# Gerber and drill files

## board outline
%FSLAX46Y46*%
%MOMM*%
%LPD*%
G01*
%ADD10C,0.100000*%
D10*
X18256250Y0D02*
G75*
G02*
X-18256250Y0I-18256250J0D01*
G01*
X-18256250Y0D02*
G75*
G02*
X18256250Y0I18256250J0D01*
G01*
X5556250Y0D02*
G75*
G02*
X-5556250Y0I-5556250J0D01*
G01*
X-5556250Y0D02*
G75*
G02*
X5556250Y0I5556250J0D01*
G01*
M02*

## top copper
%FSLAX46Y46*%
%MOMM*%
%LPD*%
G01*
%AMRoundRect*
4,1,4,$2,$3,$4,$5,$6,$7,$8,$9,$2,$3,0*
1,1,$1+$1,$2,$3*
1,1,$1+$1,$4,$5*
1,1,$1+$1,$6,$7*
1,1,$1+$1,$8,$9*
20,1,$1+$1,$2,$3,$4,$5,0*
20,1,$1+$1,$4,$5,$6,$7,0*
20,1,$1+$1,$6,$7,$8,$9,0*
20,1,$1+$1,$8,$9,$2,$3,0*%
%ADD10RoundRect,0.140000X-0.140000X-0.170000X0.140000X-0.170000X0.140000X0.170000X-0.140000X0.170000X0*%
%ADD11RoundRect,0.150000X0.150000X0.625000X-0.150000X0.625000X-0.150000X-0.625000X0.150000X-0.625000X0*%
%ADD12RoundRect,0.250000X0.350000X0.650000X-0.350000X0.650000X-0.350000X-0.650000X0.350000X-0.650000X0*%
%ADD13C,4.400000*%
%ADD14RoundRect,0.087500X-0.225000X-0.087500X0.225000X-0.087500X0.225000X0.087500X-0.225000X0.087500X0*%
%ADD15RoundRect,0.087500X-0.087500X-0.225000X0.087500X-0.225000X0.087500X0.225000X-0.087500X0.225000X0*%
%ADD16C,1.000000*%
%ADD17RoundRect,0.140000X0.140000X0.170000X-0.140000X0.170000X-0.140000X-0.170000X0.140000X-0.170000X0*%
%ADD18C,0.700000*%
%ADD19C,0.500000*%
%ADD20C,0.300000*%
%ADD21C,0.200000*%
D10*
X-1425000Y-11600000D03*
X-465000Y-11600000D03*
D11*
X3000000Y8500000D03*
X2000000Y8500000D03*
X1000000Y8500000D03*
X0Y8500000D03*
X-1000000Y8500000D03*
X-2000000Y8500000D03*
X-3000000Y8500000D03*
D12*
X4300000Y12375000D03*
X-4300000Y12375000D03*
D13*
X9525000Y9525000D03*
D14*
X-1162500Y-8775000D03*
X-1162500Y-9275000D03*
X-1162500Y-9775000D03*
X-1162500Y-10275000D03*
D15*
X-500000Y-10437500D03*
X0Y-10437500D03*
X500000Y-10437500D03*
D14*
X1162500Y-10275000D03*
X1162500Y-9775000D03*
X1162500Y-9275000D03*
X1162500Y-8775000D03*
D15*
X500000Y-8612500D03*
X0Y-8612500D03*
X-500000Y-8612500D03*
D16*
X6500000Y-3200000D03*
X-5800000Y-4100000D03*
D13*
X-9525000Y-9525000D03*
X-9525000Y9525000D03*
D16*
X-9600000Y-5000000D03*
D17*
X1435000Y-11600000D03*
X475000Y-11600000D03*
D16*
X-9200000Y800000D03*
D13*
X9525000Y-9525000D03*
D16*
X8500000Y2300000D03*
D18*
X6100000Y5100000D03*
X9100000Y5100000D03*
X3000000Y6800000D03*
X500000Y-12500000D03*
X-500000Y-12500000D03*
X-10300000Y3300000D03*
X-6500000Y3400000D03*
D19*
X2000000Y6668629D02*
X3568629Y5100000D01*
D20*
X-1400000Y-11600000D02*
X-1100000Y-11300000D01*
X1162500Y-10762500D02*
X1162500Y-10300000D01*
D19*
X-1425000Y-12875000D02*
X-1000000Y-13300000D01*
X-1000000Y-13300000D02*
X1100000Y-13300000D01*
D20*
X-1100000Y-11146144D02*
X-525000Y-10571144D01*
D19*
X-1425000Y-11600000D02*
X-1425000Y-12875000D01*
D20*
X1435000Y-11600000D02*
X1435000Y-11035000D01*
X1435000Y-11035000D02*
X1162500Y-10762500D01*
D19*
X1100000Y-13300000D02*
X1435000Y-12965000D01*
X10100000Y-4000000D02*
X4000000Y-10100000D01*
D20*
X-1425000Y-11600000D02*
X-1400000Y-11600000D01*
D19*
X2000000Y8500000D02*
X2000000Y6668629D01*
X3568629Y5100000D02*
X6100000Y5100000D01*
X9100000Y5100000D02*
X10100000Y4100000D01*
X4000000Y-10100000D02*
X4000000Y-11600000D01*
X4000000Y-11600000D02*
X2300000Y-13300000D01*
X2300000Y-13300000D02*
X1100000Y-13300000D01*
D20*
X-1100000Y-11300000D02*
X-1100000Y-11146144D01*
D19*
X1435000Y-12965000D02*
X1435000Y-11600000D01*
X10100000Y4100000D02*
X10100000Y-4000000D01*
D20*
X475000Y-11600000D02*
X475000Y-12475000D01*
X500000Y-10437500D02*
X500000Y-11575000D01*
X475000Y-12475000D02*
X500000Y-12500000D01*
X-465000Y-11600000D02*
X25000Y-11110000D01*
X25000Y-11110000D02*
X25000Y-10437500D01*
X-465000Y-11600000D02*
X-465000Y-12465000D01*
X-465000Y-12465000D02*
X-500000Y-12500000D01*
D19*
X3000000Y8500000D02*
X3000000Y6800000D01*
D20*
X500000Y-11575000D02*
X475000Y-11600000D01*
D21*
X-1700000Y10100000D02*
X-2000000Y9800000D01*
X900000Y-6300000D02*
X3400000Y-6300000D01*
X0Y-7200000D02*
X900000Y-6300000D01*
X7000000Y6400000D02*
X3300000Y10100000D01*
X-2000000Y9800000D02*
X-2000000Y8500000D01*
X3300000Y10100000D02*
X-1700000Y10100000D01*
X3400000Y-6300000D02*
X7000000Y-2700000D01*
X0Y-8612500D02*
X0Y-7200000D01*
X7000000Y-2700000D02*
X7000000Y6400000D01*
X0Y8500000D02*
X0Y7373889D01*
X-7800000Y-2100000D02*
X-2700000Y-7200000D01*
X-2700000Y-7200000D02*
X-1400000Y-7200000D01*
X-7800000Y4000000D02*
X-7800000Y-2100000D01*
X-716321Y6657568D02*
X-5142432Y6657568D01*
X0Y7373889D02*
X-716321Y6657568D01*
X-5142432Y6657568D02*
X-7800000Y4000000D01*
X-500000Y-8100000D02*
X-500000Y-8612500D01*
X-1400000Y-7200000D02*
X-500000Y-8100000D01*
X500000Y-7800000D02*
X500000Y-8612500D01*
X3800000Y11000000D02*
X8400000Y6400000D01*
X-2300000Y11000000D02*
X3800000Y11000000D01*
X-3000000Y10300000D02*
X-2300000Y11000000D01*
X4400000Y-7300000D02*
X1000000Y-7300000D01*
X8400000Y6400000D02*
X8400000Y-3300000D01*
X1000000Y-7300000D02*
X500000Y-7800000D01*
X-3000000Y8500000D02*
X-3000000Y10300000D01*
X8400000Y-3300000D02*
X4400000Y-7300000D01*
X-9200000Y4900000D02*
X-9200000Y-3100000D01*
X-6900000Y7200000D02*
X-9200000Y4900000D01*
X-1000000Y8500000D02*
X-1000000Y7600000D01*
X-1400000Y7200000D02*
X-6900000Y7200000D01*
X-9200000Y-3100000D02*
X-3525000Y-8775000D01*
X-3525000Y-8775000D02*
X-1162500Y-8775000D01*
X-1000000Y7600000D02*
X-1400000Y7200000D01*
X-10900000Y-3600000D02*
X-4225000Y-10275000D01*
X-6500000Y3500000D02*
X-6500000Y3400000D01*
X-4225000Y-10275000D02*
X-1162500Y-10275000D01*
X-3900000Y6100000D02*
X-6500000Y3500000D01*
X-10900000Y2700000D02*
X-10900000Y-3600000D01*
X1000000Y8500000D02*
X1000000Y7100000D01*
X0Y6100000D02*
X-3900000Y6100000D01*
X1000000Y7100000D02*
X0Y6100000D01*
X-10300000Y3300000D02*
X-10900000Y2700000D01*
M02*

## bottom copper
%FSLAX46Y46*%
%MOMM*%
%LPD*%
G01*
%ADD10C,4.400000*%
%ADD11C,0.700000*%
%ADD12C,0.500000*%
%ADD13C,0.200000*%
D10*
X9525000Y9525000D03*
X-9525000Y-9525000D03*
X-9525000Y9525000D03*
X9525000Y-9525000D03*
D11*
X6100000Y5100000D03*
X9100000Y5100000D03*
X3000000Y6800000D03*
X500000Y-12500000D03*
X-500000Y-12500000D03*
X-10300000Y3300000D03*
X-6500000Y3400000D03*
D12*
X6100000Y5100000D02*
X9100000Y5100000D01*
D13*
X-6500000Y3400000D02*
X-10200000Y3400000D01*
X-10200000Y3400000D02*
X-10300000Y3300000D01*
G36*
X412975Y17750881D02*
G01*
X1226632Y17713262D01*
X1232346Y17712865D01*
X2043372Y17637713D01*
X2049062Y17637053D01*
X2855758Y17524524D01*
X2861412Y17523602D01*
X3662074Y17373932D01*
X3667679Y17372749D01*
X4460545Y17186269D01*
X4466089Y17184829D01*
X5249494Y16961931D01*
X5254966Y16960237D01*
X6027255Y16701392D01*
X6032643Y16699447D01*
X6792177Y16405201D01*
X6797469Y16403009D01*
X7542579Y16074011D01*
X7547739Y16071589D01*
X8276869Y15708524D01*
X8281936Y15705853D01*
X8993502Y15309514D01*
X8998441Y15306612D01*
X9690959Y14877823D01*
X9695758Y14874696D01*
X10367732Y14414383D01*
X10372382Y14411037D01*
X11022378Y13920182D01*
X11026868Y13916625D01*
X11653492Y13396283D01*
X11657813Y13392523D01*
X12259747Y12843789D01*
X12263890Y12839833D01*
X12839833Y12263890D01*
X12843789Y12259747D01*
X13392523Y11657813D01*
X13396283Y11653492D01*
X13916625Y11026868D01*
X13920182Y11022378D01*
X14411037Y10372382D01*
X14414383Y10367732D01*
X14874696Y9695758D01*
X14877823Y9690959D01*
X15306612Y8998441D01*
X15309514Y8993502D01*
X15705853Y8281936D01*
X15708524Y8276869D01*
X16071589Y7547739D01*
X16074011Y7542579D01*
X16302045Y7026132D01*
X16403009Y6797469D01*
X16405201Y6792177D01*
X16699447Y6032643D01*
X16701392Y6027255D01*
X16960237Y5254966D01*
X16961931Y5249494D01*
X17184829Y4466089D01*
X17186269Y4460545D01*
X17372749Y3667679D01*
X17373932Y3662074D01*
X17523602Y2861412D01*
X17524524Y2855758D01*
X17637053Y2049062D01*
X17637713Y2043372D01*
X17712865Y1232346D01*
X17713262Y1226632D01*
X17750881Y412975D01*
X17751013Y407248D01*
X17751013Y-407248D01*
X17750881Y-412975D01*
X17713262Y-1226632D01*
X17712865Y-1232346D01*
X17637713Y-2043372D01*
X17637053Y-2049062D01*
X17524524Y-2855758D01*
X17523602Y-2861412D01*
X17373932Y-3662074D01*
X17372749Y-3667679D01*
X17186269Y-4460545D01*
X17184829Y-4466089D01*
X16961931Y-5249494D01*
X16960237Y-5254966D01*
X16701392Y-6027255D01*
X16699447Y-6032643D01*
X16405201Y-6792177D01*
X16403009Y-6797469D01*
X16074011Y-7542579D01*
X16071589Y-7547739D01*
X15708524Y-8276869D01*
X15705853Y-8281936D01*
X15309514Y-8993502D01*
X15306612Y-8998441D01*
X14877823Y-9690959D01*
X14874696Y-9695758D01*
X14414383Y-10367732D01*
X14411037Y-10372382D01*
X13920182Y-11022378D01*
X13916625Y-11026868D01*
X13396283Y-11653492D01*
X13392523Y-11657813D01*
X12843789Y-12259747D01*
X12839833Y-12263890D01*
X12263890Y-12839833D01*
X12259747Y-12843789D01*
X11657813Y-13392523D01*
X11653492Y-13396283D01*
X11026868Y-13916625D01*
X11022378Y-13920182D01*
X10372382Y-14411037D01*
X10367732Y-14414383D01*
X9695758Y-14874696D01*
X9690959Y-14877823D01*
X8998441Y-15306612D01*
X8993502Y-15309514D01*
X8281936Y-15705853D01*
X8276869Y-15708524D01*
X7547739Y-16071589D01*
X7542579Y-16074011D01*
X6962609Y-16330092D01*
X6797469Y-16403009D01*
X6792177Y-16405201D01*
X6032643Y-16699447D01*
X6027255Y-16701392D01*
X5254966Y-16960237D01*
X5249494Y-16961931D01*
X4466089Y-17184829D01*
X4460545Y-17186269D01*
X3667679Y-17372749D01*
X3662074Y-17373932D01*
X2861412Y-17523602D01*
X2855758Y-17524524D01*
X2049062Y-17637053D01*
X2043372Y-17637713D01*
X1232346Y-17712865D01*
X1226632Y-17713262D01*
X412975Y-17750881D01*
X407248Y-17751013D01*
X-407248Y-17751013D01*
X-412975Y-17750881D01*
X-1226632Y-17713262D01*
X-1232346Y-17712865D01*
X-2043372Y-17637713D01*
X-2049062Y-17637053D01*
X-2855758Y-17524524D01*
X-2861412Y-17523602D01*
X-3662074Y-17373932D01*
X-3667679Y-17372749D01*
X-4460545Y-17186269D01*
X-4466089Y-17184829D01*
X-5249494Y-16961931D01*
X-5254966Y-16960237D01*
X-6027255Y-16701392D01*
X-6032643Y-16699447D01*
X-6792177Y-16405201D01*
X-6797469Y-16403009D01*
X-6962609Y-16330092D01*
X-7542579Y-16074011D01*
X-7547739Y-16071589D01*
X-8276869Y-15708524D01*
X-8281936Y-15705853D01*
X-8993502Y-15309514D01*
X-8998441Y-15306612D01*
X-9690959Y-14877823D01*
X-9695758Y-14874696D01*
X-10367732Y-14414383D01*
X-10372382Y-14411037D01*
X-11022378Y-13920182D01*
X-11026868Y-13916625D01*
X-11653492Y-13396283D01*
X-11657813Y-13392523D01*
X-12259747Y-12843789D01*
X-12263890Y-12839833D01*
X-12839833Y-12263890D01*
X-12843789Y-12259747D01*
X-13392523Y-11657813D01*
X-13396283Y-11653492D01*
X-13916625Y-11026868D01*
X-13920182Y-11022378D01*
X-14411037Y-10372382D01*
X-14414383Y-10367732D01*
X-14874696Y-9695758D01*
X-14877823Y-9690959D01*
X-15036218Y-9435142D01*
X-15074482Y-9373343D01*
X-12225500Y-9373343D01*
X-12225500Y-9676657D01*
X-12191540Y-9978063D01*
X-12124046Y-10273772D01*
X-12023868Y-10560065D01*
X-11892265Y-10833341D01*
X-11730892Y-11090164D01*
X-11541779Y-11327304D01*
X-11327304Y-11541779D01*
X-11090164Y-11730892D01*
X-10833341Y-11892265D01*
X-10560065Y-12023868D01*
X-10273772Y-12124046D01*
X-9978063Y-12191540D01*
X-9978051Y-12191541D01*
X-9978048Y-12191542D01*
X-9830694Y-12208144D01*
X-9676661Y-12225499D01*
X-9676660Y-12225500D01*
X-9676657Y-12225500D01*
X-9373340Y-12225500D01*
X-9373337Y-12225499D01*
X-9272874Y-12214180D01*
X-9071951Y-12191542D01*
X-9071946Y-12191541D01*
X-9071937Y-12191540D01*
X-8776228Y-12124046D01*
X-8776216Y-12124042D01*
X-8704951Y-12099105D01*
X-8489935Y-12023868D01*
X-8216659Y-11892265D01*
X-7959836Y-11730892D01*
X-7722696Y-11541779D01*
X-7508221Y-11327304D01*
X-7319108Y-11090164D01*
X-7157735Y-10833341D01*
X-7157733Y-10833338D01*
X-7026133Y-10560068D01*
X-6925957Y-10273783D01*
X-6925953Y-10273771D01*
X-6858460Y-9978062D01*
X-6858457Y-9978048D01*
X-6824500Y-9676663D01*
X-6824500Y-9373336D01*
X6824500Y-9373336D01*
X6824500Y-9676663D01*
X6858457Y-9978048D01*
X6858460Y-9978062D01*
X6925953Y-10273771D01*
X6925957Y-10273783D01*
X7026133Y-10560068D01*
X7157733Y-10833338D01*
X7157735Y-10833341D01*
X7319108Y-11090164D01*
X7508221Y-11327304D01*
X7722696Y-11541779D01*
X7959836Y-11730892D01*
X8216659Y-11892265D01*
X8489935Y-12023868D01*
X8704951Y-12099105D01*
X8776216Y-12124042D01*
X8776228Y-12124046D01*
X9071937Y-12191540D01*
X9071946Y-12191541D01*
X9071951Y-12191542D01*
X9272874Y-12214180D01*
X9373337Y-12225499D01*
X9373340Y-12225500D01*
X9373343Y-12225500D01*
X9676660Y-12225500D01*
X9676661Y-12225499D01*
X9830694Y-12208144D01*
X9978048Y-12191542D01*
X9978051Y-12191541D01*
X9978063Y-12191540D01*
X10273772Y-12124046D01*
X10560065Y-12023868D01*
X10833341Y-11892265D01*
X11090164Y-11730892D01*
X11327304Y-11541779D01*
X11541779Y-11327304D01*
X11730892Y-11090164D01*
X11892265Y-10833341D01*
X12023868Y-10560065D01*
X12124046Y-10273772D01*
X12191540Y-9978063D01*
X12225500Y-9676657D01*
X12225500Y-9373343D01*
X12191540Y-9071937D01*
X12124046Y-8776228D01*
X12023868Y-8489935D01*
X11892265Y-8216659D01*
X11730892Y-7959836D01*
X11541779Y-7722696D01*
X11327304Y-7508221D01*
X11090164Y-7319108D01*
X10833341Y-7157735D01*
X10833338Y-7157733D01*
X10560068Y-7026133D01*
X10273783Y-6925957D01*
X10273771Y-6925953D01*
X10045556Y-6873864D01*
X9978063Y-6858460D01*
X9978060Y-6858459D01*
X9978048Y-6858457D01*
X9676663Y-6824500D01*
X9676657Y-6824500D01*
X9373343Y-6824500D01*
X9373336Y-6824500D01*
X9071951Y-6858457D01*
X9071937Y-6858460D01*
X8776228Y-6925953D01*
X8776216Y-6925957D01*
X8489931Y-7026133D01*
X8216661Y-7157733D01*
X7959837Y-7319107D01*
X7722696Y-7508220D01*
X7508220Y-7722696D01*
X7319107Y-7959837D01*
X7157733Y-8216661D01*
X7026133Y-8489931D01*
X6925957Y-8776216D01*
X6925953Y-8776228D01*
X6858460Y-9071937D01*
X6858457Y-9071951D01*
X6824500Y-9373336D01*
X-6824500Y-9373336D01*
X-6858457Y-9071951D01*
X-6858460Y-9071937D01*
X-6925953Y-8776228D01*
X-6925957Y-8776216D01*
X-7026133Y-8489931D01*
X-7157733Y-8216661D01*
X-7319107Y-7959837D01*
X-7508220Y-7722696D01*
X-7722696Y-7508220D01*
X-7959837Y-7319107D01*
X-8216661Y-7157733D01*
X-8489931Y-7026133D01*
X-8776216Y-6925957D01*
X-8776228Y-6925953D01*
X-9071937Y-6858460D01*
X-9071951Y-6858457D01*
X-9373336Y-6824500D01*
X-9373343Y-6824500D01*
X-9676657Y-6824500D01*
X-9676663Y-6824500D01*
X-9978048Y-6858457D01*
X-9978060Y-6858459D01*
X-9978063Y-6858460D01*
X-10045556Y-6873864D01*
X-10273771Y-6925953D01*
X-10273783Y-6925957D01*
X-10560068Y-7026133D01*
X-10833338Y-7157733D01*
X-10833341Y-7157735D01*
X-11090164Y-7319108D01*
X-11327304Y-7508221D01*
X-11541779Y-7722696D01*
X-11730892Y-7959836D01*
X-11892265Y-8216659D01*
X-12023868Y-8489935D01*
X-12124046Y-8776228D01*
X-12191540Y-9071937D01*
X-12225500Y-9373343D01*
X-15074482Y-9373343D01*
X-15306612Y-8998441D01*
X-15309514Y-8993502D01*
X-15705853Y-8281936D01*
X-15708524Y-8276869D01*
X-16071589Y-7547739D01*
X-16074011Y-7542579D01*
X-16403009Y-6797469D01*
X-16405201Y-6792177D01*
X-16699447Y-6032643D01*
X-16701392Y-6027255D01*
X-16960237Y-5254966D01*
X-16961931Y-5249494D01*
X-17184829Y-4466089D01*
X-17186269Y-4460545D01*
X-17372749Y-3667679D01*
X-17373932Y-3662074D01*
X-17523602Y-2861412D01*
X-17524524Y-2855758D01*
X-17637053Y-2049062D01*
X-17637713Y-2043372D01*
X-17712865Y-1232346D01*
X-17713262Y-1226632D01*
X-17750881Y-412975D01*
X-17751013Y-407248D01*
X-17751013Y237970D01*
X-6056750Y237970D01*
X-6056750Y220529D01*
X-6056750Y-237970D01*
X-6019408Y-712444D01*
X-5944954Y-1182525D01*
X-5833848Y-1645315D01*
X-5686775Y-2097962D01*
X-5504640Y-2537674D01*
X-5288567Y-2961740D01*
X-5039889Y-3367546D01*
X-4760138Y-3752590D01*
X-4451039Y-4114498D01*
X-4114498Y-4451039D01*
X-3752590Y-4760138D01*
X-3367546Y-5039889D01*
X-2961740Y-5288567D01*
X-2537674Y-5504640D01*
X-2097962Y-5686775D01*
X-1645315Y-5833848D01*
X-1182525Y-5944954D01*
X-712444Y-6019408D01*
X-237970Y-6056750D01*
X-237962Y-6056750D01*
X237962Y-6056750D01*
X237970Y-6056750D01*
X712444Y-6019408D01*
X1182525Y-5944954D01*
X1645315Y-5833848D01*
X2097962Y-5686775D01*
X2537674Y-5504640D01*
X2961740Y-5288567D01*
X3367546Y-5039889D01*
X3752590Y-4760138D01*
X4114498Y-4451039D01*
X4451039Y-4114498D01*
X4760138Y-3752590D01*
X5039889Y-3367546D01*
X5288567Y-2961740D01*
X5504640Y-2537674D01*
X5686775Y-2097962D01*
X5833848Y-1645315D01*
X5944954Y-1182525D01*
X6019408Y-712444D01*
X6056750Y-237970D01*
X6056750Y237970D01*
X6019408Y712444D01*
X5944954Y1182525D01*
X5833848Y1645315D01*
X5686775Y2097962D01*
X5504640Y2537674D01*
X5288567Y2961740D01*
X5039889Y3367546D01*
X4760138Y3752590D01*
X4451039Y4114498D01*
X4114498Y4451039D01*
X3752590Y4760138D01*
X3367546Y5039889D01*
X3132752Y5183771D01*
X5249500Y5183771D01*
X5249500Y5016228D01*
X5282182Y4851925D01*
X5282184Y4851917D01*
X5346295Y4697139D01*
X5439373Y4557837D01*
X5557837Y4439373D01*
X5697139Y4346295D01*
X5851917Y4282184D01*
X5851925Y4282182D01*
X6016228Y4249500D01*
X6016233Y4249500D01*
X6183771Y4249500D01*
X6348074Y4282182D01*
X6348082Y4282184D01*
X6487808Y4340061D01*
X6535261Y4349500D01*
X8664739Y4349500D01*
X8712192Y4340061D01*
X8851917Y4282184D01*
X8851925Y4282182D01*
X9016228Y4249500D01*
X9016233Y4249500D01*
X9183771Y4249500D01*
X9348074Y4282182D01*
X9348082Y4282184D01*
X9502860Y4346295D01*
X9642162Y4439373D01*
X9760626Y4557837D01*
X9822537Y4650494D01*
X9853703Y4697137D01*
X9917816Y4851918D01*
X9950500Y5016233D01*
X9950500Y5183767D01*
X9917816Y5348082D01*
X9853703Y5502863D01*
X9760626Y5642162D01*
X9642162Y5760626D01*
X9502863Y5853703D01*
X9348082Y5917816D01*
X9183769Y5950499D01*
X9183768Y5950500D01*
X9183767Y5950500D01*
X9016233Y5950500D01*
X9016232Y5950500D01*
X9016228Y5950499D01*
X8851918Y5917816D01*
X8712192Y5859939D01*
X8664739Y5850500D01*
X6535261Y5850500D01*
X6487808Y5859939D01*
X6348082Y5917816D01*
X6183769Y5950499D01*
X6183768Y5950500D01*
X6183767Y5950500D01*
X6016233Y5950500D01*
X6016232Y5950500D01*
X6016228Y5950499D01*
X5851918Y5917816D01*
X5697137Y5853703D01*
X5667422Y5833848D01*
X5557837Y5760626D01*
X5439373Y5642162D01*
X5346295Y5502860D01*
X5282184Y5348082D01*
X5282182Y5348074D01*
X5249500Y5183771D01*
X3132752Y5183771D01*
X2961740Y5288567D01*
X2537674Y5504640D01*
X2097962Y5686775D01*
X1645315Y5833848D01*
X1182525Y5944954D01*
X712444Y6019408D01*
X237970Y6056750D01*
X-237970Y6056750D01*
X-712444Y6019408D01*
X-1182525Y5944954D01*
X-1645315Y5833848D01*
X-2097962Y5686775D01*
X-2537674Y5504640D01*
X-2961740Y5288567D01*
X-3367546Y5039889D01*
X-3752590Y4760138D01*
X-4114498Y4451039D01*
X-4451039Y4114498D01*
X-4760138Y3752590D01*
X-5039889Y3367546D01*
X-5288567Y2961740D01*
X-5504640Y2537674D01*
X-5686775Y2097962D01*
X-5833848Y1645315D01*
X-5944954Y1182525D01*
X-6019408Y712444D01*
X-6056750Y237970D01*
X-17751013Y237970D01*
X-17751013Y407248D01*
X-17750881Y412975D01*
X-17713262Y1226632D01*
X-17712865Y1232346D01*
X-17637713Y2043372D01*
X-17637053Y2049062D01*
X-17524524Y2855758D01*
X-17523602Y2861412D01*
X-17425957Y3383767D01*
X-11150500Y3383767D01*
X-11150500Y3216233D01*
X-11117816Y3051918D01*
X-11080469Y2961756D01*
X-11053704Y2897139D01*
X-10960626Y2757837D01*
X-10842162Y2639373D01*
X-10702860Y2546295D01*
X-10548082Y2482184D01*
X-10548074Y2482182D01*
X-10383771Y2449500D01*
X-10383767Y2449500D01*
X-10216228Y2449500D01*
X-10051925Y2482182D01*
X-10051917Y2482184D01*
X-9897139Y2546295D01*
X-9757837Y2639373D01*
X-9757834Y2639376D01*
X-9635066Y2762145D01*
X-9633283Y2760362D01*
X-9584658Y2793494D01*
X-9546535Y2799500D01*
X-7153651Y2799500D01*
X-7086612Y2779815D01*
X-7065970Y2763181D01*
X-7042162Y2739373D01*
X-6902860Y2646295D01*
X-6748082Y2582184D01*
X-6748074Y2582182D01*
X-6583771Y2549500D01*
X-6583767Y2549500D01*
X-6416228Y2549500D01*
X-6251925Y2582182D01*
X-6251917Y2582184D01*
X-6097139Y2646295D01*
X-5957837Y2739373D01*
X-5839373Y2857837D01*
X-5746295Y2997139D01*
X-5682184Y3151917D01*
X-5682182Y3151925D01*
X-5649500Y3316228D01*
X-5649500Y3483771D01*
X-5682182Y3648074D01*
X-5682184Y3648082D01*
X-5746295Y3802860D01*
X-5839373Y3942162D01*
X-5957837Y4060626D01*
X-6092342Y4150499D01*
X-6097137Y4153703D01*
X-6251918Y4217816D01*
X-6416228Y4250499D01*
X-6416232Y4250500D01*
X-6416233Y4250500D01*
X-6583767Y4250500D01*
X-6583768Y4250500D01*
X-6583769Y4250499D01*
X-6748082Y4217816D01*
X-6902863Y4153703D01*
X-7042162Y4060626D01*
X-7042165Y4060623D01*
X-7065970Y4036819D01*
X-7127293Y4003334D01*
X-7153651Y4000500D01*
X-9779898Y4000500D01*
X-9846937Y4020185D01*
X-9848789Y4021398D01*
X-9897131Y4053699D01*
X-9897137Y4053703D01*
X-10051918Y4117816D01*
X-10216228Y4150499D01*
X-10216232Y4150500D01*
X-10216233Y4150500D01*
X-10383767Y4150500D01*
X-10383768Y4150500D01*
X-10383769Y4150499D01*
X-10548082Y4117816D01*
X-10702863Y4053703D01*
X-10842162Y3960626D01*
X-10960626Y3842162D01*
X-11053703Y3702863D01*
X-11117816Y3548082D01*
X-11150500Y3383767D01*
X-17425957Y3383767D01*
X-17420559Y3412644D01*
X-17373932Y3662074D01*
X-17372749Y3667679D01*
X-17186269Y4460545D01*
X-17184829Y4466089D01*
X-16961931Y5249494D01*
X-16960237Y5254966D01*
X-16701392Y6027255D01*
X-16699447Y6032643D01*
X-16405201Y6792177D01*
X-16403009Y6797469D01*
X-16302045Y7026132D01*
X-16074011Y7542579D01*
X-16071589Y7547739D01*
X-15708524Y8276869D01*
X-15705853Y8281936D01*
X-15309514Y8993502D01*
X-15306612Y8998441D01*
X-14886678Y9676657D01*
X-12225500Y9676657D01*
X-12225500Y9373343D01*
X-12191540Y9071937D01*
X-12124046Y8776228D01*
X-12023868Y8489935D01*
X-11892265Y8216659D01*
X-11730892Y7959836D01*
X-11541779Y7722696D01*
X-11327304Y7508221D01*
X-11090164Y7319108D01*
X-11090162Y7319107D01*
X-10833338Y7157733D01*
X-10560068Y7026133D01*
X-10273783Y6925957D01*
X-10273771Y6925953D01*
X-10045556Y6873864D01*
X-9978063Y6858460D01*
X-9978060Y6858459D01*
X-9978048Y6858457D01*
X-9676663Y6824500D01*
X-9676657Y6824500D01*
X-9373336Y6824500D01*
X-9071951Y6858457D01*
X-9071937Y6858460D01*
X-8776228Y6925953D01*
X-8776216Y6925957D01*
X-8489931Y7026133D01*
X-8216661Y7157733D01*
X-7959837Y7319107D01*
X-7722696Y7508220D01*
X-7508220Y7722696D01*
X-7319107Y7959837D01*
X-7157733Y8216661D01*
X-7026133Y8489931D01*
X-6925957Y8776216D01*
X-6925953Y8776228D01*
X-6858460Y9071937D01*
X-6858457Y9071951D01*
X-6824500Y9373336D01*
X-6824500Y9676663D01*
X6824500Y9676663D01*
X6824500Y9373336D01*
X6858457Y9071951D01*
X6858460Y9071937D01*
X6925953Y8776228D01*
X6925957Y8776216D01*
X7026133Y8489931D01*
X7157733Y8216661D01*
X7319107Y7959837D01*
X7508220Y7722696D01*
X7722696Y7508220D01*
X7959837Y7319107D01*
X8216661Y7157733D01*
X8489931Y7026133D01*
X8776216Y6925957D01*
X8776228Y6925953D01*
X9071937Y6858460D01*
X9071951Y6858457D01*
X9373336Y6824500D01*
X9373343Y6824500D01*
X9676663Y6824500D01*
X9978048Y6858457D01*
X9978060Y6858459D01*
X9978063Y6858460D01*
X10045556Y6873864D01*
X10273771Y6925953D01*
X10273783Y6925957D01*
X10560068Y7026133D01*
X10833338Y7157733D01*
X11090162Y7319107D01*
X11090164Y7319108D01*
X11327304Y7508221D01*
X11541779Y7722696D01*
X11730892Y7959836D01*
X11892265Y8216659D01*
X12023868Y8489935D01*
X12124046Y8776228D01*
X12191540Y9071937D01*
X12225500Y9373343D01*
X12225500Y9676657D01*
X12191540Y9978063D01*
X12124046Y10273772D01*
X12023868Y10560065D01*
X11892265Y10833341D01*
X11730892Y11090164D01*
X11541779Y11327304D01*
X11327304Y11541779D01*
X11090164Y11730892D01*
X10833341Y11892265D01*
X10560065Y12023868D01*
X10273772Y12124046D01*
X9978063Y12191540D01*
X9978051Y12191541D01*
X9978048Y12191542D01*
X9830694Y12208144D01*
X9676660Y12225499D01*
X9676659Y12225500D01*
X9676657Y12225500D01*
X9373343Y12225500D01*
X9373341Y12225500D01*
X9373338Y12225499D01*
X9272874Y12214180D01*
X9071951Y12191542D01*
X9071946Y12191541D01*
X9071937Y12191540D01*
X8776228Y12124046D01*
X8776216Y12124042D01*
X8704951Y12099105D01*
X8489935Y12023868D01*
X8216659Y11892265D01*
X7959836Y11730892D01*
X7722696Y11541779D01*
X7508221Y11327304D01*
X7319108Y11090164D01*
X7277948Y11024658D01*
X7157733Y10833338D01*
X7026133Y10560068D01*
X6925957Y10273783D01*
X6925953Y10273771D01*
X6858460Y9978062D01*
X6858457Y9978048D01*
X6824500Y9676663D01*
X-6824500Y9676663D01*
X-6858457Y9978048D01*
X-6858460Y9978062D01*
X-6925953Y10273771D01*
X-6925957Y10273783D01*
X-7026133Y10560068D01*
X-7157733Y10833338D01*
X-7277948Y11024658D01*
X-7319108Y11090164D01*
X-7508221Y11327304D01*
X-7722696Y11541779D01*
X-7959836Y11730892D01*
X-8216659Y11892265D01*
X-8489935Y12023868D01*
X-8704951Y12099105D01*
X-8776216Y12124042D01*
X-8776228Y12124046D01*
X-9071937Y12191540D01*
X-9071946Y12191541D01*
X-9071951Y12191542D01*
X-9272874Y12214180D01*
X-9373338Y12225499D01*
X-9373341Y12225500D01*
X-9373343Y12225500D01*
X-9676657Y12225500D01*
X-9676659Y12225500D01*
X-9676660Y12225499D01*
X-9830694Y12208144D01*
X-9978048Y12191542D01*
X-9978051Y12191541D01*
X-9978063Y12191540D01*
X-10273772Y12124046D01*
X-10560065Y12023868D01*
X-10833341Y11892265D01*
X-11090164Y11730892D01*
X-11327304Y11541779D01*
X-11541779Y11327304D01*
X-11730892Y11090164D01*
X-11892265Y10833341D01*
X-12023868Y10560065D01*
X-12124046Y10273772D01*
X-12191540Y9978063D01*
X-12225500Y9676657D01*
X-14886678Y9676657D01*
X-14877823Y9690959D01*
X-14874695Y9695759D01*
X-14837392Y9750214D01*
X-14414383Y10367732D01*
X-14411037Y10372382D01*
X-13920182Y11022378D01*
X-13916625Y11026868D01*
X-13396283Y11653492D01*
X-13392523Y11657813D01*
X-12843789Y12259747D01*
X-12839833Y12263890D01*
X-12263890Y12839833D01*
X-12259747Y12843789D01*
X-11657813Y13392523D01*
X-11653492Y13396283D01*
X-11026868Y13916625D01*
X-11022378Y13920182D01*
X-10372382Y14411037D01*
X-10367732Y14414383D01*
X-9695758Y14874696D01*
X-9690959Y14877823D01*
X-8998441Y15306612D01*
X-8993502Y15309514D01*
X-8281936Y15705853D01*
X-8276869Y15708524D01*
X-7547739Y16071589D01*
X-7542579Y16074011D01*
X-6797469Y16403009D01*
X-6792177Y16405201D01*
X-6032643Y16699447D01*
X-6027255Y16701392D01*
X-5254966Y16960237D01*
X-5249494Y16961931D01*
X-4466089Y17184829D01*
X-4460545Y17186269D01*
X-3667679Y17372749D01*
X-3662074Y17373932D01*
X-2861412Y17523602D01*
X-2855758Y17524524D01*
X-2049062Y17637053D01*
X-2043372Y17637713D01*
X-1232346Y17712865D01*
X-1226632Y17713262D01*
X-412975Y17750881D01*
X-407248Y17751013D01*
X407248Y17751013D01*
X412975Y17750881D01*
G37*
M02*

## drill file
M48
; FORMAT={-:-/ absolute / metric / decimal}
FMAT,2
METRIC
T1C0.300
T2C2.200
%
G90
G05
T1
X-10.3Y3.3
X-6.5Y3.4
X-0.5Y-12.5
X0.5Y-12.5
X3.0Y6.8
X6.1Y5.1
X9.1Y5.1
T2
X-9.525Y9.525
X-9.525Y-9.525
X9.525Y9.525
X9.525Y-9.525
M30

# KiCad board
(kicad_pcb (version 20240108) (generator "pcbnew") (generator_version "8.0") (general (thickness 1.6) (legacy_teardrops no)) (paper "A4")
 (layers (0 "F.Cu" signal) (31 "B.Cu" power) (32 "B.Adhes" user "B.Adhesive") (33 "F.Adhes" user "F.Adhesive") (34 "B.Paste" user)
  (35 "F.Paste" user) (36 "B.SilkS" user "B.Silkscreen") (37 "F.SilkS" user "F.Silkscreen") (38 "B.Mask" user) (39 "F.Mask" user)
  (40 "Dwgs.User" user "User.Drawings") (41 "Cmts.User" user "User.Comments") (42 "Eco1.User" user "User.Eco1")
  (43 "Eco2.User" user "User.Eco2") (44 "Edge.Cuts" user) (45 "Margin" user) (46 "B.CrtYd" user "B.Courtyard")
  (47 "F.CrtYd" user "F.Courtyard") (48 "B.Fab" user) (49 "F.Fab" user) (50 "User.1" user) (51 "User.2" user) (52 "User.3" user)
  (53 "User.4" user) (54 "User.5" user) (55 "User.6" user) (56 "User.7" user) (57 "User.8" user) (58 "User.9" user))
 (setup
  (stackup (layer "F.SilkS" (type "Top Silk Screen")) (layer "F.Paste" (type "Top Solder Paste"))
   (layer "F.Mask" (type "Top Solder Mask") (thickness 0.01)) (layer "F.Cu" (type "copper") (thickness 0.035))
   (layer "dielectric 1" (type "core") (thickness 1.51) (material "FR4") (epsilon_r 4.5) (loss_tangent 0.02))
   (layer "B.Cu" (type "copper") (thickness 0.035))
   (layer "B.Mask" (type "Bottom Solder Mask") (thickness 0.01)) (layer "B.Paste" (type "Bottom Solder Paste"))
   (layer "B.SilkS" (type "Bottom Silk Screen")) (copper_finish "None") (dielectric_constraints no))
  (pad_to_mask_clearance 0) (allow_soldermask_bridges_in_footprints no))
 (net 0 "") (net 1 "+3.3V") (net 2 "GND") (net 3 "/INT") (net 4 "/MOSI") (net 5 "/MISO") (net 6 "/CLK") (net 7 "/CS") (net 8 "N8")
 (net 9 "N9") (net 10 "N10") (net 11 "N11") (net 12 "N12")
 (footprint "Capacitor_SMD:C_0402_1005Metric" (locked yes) (layer "F.Cu") (at -0.945 11.6)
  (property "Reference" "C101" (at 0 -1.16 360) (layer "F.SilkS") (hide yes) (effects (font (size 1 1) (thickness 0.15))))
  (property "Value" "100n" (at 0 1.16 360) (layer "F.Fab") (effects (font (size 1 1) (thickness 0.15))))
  (pad "1" smd roundrect (at -0.48 0) (size 0.56 0.62) (layers "F.Cu" "F.Paste" "F.Mask") (roundrect_rratio 0.25) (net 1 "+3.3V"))
  (pad "2" smd roundrect (at 0.48 0) (size 0.56 0.62) (layers "F.Cu" "F.Paste" "F.Mask") (roundrect_rratio 0.25) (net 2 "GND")))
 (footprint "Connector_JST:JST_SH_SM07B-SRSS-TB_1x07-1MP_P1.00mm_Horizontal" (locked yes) (layer "F.Cu") (at 0 -10.5 180)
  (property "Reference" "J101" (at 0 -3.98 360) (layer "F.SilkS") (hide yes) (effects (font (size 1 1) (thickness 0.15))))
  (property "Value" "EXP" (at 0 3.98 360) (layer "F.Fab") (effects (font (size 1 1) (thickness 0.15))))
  (pad "1" smd roundrect (at -3 -2 180) (size 0.6 1.55) (layers "F.Cu" "F.Paste" "F.Mask") (roundrect_rratio 0.25) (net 2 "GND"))
  (pad "2" smd roundrect (at -2 -2 180) (size 0.6 1.55) (layers "F.Cu" "F.Paste" "F.Mask") (roundrect_rratio 0.25) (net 1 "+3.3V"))
  (pad "3" smd roundrect (at -1 -2 180) (size 0.6 1.55) (layers "F.Cu" "F.Paste" "F.Mask") (roundrect_rratio 0.25) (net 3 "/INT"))
  (pad "4" smd roundrect (at 0 -2 180) (size 0.6 1.55) (layers "F.Cu" "F.Paste" "F.Mask") (roundrect_rratio 0.25) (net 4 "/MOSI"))
  (pad "5" smd roundrect (at 1 -2 180) (size 0.6 1.55) (layers "F.Cu" "F.Paste" "F.Mask") (roundrect_rratio 0.25) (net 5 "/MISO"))
  (pad "6" smd roundrect (at 2 -2 180) (size 0.6 1.55) (layers "F.Cu" "F.Paste" "F.Mask") (roundrect_rratio 0.25) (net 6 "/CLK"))
  (pad "7" smd roundrect (at 3 -2 180) (size 0.6 1.55) (layers "F.Cu" "F.Paste" "F.Mask") (roundrect_rratio 0.25) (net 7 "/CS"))
  (pad "MP" smd roundrect (at -4.3 1.875 180) (size 1.2 1.8) (layers "F.Cu" "F.Paste" "F.Mask") (roundrect_rratio 0.208333))
  (pad "MP" smd roundrect (at 4.3 1.875 180) (size 1.2 1.8) (layers "F.Cu" "F.Paste" "F.Mask") (roundrect_rratio 0.208333)))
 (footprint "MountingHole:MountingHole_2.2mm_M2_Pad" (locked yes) (layer "F.Cu") (at 9.525 -9.525)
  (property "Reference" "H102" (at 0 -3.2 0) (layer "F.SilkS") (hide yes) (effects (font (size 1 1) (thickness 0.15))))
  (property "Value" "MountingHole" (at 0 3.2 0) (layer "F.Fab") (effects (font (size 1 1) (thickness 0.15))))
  (pad "1" thru_hole circle (at 0 0) (size 4.4 4.4) (drill 2.2) (layers "*.Cu" "*.Mask") (remove_unused_layers no)))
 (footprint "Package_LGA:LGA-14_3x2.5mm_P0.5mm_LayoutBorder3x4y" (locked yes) (layer "F.Cu") (at 0 9.525)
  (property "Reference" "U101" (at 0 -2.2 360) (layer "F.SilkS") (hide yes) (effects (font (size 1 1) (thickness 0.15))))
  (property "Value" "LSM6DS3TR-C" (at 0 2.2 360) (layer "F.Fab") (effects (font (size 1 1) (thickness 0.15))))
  (pad "1" smd roundrect (at -1.1625 -0.75) (size 0.625 0.35) (layers "F.Cu" "F.Paste" "F.Mask") (roundrect_rratio 0.25) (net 5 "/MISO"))
  (pad "2" smd roundrect (at -1.1625 -0.25) (size 0.625 0.35) (layers "F.Cu" "F.Paste" "F.Mask") (roundrect_rratio 0.25) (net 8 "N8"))
  (pad "3" smd roundrect (at -1.1625 0.25) (size 0.625 0.35) (layers "F.Cu" "F.Paste" "F.Mask") (roundrect_rratio 0.25) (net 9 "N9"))
  (pad "4" smd roundrect (at -1.1625 0.75) (size 0.625 0.35) (layers "F.Cu" "F.Paste" "F.Mask") (roundrect_rratio 0.25) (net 3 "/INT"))
  (pad "5" smd roundrect (at -0.5 0.9125) (size 0.35 0.625) (layers "F.Cu" "F.Paste" "F.Mask") (roundrect_rratio 0.25) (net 1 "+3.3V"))
  (pad "6" smd roundrect (at 0 0.9125) (size 0.35 0.625) (layers "F.Cu" "F.Paste" "F.Mask") (roundrect_rratio 0.25) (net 2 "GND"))
  (pad "7" smd roundrect (at 0.5 0.9125) (size 0.35 0.625) (layers "F.Cu" "F.Paste" "F.Mask") (roundrect_rratio 0.25) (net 2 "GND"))
  (pad "8" smd roundrect (at 1.1625 0.75) (size 0.625 0.35) (layers "F.Cu" "F.Paste" "F.Mask") (roundrect_rratio 0.25) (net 1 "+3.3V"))
  (pad "9" smd roundrect (at 1.1625 0.25) (size 0.625 0.35) (layers "F.Cu" "F.Paste" "F.Mask") (roundrect_rratio 0.25) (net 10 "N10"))
  (pad "10" smd roundrect (at 1.1625 -0.25) (size 0.625 0.35) (layers "F.Cu" "F.Paste" "F.Mask") (roundrect_rratio 0.25) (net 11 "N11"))
  (pad "11" smd roundrect (at 1.1625 -0.75) (size 0.625 0.35) (layers "F.Cu" "F.Paste" "F.Mask") (roundrect_rratio 0.25) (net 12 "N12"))
  (pad "12" smd roundrect (at 0.5 -0.9125) (size 0.35 0.625) (layers "F.Cu" "F.Paste" "F.Mask") (roundrect_rratio 0.25) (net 7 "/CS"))
  (pad "13" smd roundrect (at 0 -0.9125) (size 0.35 0.625) (layers "F.Cu" "F.Paste" "F.Mask") (roundrect_rratio 0.25) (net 6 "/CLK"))
  (pad "14" smd roundrect (at -0.5 -0.9125) (size 0.35 0.625) (layers "F.Cu" "F.Paste" "F.Mask") (roundrect_rratio 0.25) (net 4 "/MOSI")))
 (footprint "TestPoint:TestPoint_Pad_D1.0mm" (layer "F.Cu") (at 6.5 3.2)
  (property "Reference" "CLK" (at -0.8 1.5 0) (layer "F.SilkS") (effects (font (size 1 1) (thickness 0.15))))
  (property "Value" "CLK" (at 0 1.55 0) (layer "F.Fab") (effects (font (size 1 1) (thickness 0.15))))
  (pad "1" smd circle (at 0 0) (size 1 1) (layers "F.Cu" "F.Mask") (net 6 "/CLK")))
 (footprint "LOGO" (layer "F.Cu") (at 12.7 0 90)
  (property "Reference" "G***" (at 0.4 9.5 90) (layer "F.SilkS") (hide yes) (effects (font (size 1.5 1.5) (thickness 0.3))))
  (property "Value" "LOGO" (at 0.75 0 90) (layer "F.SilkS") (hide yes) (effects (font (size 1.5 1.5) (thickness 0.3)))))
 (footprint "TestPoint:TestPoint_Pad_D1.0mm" (layer "F.Cu") (at -5.8 4.1)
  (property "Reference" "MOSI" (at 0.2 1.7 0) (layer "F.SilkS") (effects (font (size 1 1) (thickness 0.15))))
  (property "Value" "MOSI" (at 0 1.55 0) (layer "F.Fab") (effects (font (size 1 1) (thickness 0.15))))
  (pad "1" smd circle (at 0 0) (size 1 1) (layers "F.Cu" "F.Mask") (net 4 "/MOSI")))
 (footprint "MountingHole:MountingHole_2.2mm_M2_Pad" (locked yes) (layer "F.Cu") (at -9.525 9.525)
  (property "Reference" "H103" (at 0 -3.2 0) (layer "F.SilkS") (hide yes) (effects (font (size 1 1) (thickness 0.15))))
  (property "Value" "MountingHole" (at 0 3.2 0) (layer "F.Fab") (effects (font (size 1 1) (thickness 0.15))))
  (pad "1" thru_hole circle (at 0 0) (size 4.4 4.4) (drill 2.2) (layers "*.Cu" "*.Mask") (remove_unused_layers no)))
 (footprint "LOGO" (layer "F.Cu") (at -14.3 0 -90)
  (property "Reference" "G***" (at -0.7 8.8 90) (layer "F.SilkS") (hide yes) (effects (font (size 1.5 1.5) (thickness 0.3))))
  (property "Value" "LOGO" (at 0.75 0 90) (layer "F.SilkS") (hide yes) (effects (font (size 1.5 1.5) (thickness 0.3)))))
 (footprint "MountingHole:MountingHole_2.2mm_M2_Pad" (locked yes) (layer "F.Cu") (at -9.525 -9.525)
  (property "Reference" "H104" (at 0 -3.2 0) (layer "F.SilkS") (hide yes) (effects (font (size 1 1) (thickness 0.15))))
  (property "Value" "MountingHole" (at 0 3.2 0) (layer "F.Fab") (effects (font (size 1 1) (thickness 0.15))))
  (pad "1" thru_hole circle (at 0 0) (size 4.4 4.4) (drill 2.2) (layers "*.Cu" "*.Mask") (remove_unused_layers no)))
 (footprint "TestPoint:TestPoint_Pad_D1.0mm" (layer "F.Cu") (at -9.6 5)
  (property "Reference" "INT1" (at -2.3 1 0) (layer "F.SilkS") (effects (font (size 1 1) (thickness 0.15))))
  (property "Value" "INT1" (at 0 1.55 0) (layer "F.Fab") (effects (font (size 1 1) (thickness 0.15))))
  (pad "1" smd circle (at 0 0) (size 1 1) (layers "F.Cu" "F.Mask") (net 3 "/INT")))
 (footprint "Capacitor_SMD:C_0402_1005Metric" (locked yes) (layer "F.Cu") (at 0.955 11.6 180)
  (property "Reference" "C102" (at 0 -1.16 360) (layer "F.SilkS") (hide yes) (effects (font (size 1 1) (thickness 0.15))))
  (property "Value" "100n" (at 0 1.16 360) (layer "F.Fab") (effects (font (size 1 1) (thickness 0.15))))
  (pad "1" smd roundrect (at -0.48 0 180) (size 0.56 0.62) (layers "F.Cu" "F.Paste" "F.Mask") (roundrect_rratio 0.25) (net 1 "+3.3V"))
  (pad "2" smd roundrect (at 0.48 0 180) (size 0.56 0.62) (layers "F.Cu" "F.Paste" "F.Mask") (roundrect_rratio 0.25) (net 2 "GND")))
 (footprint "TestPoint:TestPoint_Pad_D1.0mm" (layer "F.Cu") (at -9.2 -0.8)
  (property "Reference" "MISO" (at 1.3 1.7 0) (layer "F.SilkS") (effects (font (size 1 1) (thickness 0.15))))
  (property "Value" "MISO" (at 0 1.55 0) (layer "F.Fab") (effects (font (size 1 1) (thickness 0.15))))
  (pad "1" smd circle (at 0 0) (size 1 1) (layers "F.Cu" "F.Mask") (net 5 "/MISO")))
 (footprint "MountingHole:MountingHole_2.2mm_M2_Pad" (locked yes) (layer "F.Cu") (at 9.525 9.525)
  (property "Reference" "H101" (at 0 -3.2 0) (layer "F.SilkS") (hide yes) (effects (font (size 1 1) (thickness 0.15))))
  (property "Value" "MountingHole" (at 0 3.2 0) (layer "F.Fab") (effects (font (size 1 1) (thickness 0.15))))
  (pad "1" thru_hole circle (at 0 0) (size 4.4 4.4) (drill 2.2) (layers "*.Cu" "*.Mask") (remove_unused_layers no)))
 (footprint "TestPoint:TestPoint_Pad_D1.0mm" (layer "F.Cu") (at 8.5 -2.3)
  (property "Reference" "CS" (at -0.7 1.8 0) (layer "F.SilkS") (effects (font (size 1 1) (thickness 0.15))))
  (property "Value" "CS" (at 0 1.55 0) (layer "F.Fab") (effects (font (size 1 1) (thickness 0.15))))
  (pad "1" smd circle (at 0 0) (size 1 1) (layers "F.Cu" "F.Mask") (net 7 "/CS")))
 (gr_circle (center 0 0) (end 18.25625 0) (stroke (width 0.1) (type default)) (fill none) (layer "Edge.Cuts"))
 (gr_circle (center 0 0) (end 5.55625 0) (stroke (width 0.1) (type default)) (fill none) (layer "Edge.Cuts"))
 (segment (start 2 -6.668629) (end 3.568629 -5.1) (width 0.5) (layer "F.Cu") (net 1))
 (segment (start -1.4 11.6) (end -1.1 11.3) (width 0.3) (layer "F.Cu") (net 1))
 (segment (start 1.1625 10.7625) (end 1.1625 10.3) (width 0.3) (layer "F.Cu") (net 1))
 (segment (start -1.425 12.875) (end -1 13.3) (width 0.5) (layer "F.Cu") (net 1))
 (segment (start -1 13.3) (end 1.1 13.3) (width 0.5) (layer "F.Cu") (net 1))
 (segment (start -1.1 11.146144) (end -0.525 10.571144) (width 0.3) (layer "F.Cu") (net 1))
 (segment (start -1.425 11.6) (end -1.425 12.875) (width 0.5) (layer "F.Cu") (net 1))
 (segment (start 1.435 11.6) (end 1.435 11.035) (width 0.3) (layer "F.Cu") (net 1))
 (segment (start 1.435 11.035) (end 1.1625 10.7625) (width 0.3) (layer "F.Cu") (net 1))
 (segment (start 1.1 13.3) (end 1.435 12.965) (width 0.5) (layer "F.Cu") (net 1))
 (segment (start 10.1 4) (end 4 10.1) (width 0.5) (layer "F.Cu") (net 1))
 (segment (start -1.425 11.6) (end -1.4 11.6) (width 0.3) (layer "F.Cu") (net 1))
 (segment (start 2 -8.5) (end 2 -6.668629) (width 0.5) (layer "F.Cu") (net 1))
 (segment (start 3.568629 -5.1) (end 6.1 -5.1) (width 0.5) (layer "F.Cu") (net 1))
 (segment (start 9.1 -5.1) (end 10.1 -4.1) (width 0.5) (layer "F.Cu") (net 1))
 (segment (start 4 10.1) (end 4 11.6) (width 0.5) (layer "F.Cu") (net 1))
 (segment (start 4 11.6) (end 2.3 13.3) (width 0.5) (layer "F.Cu") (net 1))
 (segment (start 2.3 13.3) (end 1.1 13.3) (width 0.5) (layer "F.Cu") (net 1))
 (segment (start -1.1 11.3) (end -1.1 11.146144) (width 0.3) (layer "F.Cu") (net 1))
 (segment (start 1.435 12.965) (end 1.435 11.6) (width 0.5) (layer "F.Cu") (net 1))
 (segment (start 10.1 -4.1) (end 10.1 4) (width 0.5) (layer "F.Cu") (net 1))
 (via (at 6.1 -5.1) (size 0.7) (drill 0.3) (layers "F.Cu" "B.Cu") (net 1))
 (via (at 9.1 -5.1) (size 0.7) (drill 0.3) (layers "F.Cu" "B.Cu") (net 1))
 (segment (start 6.1 -5.1) (end 9.1 -5.1) (width 0.5) (layer "B.Cu") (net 1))
 (segment (start 0.475 11.6) (end 0.475 12.475) (width 0.3) (layer "F.Cu") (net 2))
 (segment (start 0.5 10.4375) (end 0.5 11.575) (width 0.3) (layer "F.Cu") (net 2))
 (segment (start 0.475 12.475) (end 0.5 12.5) (width 0.3) (layer "F.Cu") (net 2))
 (segment (start -0.465 11.6) (end 0.025 11.11) (width 0.3) (layer "F.Cu") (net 2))
 (segment (start 0.025 11.11) (end 0.025 10.4375) (width 0.3) (layer "F.Cu") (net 2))
 (segment (start -0.465 11.6) (end -0.465 12.465) (width 0.3) (layer "F.Cu") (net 2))
 (segment (start -0.465 12.465) (end -0.5 12.5) (width 0.3) (layer "F.Cu") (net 2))
 (segment (start 3 -8.5) (end 3 -6.8) (width 0.5) (layer "F.Cu") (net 2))
 (segment (start 0.5 11.575) (end 0.475 11.6) (width 0.3) (layer "F.Cu") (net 2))
 (via (at 3 -6.8) (size 0.7) (drill 0.3) (layers "F.Cu" "B.Cu") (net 2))
 (via (at 0.5 12.5) (size 0.7) (drill 0.3) (layers "F.Cu" "B.Cu") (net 2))
 (via (at -0.5 12.5) (size 0.7) (drill 0.3) (layers "F.Cu" "B.Cu") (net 2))
 (segment (start -1.7 -10.1) (end -2 -9.8) (width 0.2) (layer "F.Cu") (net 6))
 (segment (start 0.9 6.3) (end 3.4 6.3) (width 0.2) (layer "F.Cu") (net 6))
 (segment (start 0 7.2) (end 0.9 6.3) (width 0.2) (layer "F.Cu") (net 6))
 (segment (start 7 -6.4) (end 3.3 -10.1) (width 0.2) (layer "F.Cu") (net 6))
 (segment (start -2 -9.8) (end -2 -8.5) (width 0.2) (layer "F.Cu") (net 6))
 (segment (start 3.3 -10.1) (end -1.7 -10.1) (width 0.2) (layer "F.Cu") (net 6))
 (segment (start 3.4 6.3) (end 7 2.7) (width 0.2) (layer "F.Cu") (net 6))
 (segment (start 0 8.6125) (end 0 7.2) (width 0.2) (layer "F.Cu") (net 6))
 (segment (start 7 2.7) (end 7 -6.4) (width 0.2) (layer "F.Cu") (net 6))
 (segment (start 0 -8.5) (end 0 -7.373889) (width 0.2) (layer "F.Cu") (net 4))
 (segment (start -7.8 2.1) (end -2.7 7.2) (width 0.2) (layer "F.Cu") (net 4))
 (segment (start -2.7 7.2) (end -1.4 7.2) (width 0.2) (layer "F.Cu") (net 4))
 (segment (start -7.8 -4) (end -7.8 2.1) (width 0.2) (layer "F.Cu") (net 4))
 (segment (start -0.716321 -6.657568) (end -5.142432 -6.657568) (width 0.2) (layer "F.Cu") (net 4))
 (segment (start 0 -7.373889) (end -0.716321 -6.657568) (width 0.2) (layer "F.Cu") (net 4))
 (segment (start -5.142432 -6.657568) (end -7.8 -4) (width 0.2) (layer "F.Cu") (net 4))
 (segment (start -0.5 8.1) (end -0.5 8.6125) (width 0.2) (layer "F.Cu") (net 4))
 (segment (start -1.4 7.2) (end -0.5 8.1) (width 0.2) (layer "F.Cu") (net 4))
 (segment (start 0.5 7.8) (end 0.5 8.6125) (width 0.2) (layer "F.Cu") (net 7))
 (segment (start 3.8 -11) (end 8.4 -6.4) (width 0.2) (layer "F.Cu") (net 7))
 (segment (start -2.3 -11) (end 3.8 -11) (width 0.2) (layer "F.Cu") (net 7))
 (segment (start -3 -10.3) (end -2.3 -11) (width 0.2) (layer "F.Cu") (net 7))
 (segment (start 4.4 7.3) (end 1 7.3) (width 0.2) (layer "F.Cu") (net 7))
 (segment (start 8.4 -6.4) (end 8.4 3.3) (width 0.2) (layer "F.Cu") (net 7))
 (segment (start 1 7.3) (end 0.5 7.8) (width 0.2) (layer "F.Cu") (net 7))
 (segment (start -3 -8.5) (end -3 -10.3) (width 0.2) (layer "F.Cu") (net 7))
 (segment (start 8.4 3.3) (end 4.4 7.3) (width 0.2) (layer "F.Cu") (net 7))
 (segment (start -9.2 -4.9) (end -9.2 3.1) (width 0.2) (layer "F.Cu") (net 5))
 (segment (start -6.9 -7.2) (end -9.2 -4.9) (width 0.2) (layer "F.Cu") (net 5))
 (segment (start -1 -8.5) (end -1 -7.6) (width 0.2) (layer "F.Cu") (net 5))
 (segment (start -1.4 -7.2) (end -6.9 -7.2) (width 0.2) (layer "F.Cu") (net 5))
 (segment (start -9.2 3.1) (end -3.525 8.775) (width 0.2) (layer "F.Cu") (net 5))
 (segment (start -3.525 8.775) (end -1.1625 8.775) (width 0.2) (layer "F.Cu") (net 5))
 (segment (start -1 -7.6) (end -1.4 -7.2) (width 0.2) (layer "F.Cu") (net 5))
 (segment (start -10.9 3.6) (end -4.225 10.275) (width 0.2) (layer "F.Cu") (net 3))
 (segment (start -6.5 -3.5) (end -6.5 -3.4) (width 0.2) (layer "F.Cu") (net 3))
 (segment (start -4.225 10.275) (end -1.1625 10.275) (width 0.2) (layer "F.Cu") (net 3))
 (segment (start -3.9 -6.1) (end -6.5 -3.5) (width 0.2) (layer "F.Cu") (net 3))
 (segment (start -10.9 -2.7) (end -10.9 3.6) (width 0.2) (layer "F.Cu") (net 3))
 (segment (start 1 -8.5) (end 1 -7.1) (width 0.2) (layer "F.Cu") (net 3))
 (segment (start 0 -6.1) (end -3.9 -6.1) (width 0.2) (layer "F.Cu") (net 3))
 (segment (start 1 -7.1) (end 0 -6.1) (width 0.2) (layer "F.Cu") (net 3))
 (segment (start -10.3 -3.3) (end -10.9 -2.7) (width 0.2) (layer "F.Cu") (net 3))
 (via (at -10.3 -3.3) (size 0.7) (drill 0.3) (layers "F.Cu" "B.Cu") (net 3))
 (via (at -6.5 -3.4) (size 0.7) (drill 0.3) (layers "F.Cu" "B.Cu") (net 3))
 (segment (start -6.5 -3.4) (end -10.2 -3.4) (width 0.2) (layer "B.Cu") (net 3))
 (segment (start -10.2 -3.4) (end -10.3 -3.3) (width 0.2) (layer "B.Cu") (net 3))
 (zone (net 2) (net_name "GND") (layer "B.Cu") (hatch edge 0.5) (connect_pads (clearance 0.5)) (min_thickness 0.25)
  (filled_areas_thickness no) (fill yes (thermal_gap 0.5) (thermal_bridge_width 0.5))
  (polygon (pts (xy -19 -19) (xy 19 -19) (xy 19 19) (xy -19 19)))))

